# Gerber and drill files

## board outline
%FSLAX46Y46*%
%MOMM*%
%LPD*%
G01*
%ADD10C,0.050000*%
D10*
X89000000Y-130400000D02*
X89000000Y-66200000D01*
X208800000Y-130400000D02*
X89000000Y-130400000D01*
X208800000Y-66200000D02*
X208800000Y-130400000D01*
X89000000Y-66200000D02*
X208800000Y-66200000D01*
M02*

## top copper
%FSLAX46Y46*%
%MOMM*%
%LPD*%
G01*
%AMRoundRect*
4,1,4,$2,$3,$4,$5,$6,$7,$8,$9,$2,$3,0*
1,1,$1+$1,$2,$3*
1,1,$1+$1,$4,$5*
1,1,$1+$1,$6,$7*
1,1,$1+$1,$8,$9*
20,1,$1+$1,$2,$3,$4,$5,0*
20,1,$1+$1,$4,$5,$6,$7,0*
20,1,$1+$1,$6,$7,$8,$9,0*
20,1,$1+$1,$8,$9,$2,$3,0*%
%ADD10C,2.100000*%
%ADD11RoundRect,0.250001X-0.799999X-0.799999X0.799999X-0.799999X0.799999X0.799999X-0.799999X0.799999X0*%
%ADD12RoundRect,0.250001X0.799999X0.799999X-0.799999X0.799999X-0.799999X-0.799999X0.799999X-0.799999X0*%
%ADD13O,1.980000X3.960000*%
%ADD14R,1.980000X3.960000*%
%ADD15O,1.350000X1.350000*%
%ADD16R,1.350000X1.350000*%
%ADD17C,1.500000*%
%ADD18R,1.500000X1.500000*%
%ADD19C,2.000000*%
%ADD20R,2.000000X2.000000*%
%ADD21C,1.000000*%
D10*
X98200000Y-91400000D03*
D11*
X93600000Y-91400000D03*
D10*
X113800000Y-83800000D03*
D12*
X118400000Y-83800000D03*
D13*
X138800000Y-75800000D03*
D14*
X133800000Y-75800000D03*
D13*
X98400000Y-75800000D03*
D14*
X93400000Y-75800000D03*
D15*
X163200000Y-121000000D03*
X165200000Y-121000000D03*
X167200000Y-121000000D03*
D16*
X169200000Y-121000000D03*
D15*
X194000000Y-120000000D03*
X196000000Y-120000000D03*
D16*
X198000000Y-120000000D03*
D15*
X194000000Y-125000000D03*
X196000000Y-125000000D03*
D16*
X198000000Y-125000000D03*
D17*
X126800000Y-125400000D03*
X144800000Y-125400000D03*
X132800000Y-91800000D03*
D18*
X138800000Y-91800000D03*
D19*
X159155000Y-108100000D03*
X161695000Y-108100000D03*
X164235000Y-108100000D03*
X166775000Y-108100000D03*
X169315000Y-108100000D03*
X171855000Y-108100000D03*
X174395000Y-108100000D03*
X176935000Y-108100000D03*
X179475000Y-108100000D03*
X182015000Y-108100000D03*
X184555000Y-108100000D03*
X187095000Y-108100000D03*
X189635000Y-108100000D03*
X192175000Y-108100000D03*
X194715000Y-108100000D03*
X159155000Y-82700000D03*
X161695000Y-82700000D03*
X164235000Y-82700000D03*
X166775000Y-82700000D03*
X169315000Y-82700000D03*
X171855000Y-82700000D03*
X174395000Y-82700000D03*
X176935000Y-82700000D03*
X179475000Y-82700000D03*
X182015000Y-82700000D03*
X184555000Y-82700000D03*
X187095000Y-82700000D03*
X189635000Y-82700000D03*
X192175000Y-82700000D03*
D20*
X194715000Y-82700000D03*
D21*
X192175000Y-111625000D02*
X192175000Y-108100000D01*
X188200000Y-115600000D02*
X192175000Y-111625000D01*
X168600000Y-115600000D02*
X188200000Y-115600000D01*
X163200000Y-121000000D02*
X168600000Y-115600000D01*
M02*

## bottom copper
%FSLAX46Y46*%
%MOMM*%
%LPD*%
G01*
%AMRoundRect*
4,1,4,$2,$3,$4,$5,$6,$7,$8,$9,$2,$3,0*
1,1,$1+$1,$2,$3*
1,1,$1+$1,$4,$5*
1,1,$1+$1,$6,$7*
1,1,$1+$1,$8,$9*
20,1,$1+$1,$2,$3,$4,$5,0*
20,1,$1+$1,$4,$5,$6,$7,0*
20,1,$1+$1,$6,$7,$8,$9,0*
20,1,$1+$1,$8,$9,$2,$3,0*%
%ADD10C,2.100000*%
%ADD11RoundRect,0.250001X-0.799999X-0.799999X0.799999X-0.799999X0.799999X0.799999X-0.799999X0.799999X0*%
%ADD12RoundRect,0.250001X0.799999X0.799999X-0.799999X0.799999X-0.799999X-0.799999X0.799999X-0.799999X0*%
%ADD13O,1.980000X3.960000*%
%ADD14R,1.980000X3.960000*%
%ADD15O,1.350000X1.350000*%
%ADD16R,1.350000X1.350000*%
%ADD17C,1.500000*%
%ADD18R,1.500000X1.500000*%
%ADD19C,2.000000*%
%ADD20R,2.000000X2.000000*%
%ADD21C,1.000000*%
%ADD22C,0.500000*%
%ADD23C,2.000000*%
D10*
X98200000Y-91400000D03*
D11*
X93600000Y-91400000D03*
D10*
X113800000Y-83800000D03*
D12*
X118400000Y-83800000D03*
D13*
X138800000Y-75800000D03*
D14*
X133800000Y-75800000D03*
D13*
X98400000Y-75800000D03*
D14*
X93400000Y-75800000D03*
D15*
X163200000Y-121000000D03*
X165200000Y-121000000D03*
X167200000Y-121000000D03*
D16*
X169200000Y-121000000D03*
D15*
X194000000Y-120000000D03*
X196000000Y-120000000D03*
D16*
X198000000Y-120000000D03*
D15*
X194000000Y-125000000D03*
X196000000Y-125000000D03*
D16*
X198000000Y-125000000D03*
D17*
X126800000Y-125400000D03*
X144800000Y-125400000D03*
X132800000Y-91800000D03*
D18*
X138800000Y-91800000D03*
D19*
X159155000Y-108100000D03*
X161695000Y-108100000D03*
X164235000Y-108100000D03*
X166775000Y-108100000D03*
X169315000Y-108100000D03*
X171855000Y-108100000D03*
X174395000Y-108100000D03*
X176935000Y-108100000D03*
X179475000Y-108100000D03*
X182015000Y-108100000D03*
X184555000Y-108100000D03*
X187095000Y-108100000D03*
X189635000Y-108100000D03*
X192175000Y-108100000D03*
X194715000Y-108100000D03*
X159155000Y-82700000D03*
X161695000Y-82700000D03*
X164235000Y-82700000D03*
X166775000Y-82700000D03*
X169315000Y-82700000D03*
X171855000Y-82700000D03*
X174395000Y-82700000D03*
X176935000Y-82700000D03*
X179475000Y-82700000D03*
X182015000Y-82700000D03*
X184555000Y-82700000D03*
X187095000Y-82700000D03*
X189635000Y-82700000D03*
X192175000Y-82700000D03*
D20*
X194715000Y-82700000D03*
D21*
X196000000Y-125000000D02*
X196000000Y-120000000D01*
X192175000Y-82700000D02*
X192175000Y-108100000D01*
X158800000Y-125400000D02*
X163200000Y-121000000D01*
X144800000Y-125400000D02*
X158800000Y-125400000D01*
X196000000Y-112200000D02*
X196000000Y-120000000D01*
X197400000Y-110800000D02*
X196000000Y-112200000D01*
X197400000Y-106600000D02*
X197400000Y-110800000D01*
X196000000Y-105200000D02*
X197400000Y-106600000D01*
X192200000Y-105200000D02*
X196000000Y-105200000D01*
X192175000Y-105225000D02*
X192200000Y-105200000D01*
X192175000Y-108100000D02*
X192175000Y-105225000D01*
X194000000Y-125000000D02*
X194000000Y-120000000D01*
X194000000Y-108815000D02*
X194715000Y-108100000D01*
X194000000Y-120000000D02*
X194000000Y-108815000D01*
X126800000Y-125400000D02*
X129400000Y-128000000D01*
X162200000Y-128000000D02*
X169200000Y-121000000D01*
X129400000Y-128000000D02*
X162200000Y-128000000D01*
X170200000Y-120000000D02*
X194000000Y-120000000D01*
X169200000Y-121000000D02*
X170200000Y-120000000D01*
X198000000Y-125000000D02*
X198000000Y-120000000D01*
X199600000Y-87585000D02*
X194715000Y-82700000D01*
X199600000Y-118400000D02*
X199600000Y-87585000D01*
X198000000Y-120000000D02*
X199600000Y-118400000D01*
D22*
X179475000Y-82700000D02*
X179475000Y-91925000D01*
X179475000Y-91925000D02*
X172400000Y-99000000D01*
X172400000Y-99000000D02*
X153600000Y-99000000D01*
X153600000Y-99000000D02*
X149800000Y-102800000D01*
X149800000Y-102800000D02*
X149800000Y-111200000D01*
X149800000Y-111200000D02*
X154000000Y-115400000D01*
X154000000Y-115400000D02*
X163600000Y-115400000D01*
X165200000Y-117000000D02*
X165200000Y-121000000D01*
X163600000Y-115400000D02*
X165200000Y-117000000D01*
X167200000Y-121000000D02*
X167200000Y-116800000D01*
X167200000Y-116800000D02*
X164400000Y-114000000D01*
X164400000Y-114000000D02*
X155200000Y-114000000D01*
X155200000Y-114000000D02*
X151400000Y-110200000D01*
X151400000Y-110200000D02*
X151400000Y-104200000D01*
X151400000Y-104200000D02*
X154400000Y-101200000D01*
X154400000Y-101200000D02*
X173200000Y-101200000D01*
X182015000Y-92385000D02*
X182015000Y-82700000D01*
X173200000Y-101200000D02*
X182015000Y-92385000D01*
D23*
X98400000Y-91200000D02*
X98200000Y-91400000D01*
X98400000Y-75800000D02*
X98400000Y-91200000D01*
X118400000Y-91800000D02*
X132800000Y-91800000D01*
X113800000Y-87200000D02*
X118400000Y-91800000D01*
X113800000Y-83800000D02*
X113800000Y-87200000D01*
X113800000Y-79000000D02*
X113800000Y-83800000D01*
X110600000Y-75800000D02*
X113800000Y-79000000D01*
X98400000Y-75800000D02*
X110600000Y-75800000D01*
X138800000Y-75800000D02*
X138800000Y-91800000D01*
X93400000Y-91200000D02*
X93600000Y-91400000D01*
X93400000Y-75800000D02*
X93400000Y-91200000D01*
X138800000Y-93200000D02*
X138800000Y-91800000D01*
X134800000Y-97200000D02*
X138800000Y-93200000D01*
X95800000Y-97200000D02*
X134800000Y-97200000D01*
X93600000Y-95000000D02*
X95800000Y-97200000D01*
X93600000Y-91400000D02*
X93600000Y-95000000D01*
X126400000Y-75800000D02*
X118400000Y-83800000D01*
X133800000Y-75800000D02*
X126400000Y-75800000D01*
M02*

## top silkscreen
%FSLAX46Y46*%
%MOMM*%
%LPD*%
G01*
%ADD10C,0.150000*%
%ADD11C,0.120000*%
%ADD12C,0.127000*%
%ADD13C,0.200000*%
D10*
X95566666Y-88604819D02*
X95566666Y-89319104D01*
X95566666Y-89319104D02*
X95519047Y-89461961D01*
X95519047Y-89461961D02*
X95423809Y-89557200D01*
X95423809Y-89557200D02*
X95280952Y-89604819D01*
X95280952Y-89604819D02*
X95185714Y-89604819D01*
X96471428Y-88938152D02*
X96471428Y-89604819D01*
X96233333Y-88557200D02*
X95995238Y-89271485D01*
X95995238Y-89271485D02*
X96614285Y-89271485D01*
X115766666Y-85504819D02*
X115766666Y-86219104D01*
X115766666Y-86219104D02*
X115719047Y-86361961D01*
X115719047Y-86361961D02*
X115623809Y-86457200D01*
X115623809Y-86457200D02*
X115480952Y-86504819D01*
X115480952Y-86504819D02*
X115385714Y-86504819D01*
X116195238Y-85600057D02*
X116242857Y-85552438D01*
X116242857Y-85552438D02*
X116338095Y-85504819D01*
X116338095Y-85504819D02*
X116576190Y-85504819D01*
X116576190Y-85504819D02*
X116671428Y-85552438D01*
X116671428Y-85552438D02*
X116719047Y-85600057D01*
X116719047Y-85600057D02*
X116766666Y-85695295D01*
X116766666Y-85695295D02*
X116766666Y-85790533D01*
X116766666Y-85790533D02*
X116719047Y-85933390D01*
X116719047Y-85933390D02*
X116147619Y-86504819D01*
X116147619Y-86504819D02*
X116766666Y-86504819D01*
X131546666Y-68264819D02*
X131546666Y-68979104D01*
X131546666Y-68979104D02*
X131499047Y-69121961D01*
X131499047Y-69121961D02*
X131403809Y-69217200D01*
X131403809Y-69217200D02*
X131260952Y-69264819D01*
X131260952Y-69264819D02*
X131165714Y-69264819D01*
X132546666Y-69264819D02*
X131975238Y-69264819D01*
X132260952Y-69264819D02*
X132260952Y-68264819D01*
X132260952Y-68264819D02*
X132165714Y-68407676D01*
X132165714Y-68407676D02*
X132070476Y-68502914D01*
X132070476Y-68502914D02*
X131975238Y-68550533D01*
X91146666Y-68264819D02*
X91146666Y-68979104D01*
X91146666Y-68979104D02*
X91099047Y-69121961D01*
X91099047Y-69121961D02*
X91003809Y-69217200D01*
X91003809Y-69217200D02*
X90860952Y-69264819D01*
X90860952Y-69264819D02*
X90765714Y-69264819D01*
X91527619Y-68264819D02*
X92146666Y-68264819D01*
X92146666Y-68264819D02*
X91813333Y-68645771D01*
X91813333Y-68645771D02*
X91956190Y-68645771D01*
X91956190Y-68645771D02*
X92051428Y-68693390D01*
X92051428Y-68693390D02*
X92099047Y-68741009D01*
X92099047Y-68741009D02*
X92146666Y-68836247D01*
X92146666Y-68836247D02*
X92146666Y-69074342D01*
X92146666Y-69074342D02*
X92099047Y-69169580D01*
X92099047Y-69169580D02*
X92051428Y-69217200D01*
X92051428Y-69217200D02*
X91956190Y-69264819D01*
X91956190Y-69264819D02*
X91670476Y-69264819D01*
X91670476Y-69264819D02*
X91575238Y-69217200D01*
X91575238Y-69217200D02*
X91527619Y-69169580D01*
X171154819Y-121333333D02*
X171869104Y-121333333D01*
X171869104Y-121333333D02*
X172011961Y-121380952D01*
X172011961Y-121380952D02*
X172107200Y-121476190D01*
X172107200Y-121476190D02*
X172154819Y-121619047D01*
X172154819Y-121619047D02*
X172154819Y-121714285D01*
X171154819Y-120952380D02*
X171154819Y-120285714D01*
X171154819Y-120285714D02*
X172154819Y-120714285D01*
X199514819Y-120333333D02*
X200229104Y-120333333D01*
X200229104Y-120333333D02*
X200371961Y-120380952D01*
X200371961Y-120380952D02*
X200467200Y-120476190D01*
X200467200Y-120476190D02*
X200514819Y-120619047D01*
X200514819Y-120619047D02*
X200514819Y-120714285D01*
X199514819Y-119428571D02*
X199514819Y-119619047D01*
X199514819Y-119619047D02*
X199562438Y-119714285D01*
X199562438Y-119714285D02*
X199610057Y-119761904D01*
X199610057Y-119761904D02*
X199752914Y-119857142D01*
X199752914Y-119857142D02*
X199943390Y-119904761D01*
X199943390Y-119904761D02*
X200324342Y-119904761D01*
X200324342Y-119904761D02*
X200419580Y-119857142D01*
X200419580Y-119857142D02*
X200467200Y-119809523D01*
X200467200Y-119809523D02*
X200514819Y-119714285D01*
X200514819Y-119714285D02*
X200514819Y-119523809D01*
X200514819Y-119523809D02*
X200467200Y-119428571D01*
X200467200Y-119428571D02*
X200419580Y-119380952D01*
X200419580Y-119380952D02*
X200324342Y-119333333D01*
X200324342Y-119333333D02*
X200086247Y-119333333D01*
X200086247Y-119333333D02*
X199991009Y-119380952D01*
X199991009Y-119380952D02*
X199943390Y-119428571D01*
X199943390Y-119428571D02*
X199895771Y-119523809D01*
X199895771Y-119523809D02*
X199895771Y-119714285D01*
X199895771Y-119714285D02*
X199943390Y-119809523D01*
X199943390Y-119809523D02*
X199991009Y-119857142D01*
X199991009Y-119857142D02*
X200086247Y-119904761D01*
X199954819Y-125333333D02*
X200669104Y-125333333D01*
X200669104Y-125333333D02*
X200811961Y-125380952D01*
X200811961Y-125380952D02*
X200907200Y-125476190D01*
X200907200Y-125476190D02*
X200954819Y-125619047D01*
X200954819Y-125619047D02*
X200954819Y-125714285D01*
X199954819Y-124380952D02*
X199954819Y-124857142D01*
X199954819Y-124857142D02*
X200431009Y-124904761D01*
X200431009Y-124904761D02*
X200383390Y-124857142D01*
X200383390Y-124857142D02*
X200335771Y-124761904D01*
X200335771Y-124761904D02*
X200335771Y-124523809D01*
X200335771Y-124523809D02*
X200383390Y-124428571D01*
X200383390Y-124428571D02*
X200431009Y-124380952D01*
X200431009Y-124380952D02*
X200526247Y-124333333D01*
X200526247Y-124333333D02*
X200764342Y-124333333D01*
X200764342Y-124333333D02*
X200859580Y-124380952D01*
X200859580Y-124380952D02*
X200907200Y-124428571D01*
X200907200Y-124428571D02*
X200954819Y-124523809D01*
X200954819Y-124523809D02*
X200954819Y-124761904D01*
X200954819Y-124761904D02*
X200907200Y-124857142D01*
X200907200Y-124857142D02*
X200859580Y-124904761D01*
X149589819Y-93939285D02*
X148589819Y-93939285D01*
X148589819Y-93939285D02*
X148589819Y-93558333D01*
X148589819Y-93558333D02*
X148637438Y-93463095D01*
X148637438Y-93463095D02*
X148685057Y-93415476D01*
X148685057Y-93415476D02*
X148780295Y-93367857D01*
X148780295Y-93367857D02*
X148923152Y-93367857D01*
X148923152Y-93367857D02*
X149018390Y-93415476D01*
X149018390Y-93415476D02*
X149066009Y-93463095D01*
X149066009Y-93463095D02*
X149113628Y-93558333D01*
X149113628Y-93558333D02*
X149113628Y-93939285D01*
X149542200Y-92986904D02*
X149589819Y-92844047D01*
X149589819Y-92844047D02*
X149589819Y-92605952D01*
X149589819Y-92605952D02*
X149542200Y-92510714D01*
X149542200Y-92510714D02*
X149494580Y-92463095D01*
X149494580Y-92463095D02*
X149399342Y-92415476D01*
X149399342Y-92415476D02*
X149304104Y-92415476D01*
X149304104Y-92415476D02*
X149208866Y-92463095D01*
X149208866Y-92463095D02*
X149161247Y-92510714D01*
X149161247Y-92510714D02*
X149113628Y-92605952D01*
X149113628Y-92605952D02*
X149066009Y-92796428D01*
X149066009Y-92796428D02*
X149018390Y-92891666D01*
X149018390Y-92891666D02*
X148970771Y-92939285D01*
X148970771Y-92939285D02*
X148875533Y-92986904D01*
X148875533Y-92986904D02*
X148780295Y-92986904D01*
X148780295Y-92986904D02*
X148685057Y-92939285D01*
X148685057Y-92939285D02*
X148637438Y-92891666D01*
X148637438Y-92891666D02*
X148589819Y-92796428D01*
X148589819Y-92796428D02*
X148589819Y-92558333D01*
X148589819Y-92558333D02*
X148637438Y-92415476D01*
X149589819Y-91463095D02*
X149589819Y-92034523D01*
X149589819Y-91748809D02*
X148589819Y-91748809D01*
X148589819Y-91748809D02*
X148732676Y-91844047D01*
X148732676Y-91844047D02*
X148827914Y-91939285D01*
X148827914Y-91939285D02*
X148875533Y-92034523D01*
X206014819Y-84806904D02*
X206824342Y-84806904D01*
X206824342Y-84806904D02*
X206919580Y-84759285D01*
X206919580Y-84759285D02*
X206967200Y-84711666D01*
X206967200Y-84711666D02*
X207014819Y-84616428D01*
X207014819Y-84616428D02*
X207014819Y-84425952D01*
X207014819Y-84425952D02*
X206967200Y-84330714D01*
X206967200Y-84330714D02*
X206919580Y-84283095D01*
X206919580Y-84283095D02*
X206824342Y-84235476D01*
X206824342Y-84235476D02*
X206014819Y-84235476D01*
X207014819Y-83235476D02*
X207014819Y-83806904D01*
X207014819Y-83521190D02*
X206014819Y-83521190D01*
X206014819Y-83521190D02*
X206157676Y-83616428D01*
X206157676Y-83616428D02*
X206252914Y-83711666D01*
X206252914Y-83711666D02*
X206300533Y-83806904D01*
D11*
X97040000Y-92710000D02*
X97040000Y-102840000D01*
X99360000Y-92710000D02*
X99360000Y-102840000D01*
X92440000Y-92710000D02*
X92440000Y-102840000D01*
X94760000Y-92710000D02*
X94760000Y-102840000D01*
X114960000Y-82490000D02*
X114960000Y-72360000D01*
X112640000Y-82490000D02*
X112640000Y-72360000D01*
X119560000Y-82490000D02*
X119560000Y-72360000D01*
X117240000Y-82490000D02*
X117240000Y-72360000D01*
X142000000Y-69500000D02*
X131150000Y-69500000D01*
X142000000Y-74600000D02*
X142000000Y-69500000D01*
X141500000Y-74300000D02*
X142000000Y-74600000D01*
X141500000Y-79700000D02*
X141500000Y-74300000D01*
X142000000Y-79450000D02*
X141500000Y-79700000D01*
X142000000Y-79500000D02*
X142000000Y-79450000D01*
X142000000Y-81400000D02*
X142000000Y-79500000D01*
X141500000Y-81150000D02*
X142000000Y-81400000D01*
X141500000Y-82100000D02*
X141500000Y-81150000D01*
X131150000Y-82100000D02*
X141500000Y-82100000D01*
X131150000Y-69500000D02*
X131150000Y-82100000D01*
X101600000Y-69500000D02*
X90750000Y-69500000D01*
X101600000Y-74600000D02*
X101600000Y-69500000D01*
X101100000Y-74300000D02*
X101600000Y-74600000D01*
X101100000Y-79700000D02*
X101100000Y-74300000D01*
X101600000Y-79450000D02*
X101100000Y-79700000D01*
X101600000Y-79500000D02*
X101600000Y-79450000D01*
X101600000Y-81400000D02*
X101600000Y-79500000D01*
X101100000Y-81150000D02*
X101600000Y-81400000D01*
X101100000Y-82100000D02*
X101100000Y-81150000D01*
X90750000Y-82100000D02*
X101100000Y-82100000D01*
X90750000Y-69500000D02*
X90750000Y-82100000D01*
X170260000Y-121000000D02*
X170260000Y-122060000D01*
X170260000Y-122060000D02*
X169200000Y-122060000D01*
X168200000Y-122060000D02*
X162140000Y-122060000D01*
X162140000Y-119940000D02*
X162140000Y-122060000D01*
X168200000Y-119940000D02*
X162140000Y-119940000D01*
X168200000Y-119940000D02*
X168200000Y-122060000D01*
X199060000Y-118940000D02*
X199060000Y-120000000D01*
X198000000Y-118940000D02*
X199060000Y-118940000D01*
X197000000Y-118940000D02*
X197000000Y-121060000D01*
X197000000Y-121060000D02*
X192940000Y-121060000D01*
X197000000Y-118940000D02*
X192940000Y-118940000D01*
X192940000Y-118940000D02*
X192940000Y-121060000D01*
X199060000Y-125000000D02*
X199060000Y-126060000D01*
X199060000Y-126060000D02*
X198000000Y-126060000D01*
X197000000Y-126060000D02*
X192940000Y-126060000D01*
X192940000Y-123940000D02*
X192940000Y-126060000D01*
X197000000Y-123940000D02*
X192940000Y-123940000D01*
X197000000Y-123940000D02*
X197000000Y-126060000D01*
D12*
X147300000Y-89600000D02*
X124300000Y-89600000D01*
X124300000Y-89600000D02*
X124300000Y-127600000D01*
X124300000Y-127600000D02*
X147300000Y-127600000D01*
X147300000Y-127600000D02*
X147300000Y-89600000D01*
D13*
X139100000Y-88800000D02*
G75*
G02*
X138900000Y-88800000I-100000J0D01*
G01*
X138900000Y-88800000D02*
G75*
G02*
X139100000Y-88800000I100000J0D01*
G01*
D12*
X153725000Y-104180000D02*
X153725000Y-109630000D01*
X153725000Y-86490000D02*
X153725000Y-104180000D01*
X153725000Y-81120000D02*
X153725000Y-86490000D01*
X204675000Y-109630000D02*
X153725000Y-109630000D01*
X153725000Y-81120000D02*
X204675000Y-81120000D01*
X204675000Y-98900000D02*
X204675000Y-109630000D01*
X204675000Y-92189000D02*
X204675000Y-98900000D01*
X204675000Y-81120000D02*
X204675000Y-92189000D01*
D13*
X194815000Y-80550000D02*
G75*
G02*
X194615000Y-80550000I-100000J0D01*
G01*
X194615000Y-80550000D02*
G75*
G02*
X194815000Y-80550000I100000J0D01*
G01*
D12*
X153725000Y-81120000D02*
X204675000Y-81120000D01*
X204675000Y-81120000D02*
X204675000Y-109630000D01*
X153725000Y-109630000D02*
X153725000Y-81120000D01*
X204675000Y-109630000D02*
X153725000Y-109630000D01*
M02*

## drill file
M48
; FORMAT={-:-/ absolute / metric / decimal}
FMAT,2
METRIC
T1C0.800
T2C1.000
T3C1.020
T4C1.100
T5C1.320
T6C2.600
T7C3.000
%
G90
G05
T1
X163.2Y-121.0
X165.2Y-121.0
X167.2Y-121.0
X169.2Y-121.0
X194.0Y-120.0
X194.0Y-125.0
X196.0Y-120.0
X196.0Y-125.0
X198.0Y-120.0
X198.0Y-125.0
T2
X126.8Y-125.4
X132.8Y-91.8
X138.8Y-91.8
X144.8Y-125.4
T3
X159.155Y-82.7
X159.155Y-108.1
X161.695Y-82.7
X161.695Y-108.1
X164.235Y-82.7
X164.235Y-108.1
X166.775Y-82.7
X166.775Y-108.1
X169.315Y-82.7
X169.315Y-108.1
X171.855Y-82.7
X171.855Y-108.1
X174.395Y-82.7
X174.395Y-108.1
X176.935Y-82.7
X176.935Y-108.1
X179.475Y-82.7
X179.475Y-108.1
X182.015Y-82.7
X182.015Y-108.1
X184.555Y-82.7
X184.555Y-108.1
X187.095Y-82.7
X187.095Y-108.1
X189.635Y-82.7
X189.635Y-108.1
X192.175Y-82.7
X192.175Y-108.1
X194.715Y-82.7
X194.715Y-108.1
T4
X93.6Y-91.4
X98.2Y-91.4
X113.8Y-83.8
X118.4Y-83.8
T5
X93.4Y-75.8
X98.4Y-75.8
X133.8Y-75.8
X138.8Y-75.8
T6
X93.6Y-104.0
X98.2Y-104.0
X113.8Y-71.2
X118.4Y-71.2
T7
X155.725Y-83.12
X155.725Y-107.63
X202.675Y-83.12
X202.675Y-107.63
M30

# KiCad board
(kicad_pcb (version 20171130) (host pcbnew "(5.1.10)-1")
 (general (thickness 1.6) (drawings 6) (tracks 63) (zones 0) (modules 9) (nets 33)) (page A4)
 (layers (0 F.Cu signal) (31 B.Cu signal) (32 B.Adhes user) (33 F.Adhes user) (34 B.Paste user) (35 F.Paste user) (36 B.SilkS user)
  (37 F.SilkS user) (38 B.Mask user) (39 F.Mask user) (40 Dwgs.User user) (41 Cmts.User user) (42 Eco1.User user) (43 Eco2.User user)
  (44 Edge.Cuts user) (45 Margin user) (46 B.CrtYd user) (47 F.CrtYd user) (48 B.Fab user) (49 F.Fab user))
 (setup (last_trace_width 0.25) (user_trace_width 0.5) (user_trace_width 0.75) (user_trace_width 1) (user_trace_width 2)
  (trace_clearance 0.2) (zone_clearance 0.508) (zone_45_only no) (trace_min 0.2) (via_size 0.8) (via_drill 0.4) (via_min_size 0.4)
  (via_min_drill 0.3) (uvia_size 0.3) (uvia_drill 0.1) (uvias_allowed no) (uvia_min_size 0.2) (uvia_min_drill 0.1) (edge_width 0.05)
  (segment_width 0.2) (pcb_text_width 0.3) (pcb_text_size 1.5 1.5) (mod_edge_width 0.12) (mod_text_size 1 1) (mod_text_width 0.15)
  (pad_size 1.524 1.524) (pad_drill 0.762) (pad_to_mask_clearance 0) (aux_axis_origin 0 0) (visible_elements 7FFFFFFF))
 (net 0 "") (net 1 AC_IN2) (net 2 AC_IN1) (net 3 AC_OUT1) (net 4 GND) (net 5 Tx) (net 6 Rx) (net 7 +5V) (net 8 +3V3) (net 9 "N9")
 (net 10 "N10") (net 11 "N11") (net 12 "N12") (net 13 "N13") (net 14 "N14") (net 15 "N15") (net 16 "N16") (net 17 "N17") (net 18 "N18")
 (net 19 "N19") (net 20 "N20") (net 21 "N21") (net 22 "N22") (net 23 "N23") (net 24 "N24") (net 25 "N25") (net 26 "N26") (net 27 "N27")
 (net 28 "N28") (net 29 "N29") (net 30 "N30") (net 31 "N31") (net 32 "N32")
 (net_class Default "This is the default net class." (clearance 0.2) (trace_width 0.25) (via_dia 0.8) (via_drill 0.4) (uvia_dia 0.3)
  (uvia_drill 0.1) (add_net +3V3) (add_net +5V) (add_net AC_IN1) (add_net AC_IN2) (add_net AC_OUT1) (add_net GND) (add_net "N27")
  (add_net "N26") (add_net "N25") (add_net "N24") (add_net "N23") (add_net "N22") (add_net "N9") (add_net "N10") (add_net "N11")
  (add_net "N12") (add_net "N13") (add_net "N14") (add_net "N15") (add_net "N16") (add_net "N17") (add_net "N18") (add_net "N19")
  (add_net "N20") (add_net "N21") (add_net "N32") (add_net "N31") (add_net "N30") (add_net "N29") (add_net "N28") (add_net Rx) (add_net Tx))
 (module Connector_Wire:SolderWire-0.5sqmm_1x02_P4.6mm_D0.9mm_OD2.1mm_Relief (layer F.Cu) (at 93.6 91.4)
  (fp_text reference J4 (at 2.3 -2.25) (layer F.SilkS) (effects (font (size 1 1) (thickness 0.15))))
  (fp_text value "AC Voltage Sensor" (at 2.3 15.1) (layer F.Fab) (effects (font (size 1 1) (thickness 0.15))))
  (fp_line (start 3.44 1.31) (end 3.44 11.44) (layer F.SilkS) (width 0.12))
  (fp_line (start 5.76 1.31) (end 5.76 11.44) (layer F.SilkS) (width 0.12))
  (fp_line (start -1.16 1.31) (end -1.16 11.44) (layer F.SilkS) (width 0.12))
  (fp_line (start 1.16 1.31) (end 1.16 11.44) (layer F.SilkS) (width 0.12))
  (pad "" np_thru_hole circle (at 4.6 12.6) (size 2.6 2.6) (drill 2.6) (layers *.Cu *.Mask))
  (pad "" np_thru_hole circle (at 0 12.6) (size 2.6 2.6) (drill 2.6) (layers *.Cu *.Mask))
  (pad 2 thru_hole circle (at 4.6 0) (size 2.1 2.1) (drill 1.1) (layers *.Cu *.Mask) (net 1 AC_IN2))
  (pad 1 thru_hole roundrect (at 0 0) (size 2.1 2.1) (drill 1.1) (layers *.Cu *.Mask) (roundrect_rratio 0.119048) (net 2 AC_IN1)))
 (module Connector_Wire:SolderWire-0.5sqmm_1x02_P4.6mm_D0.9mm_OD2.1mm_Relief (layer F.Cu) (at 118.4 83.8 180)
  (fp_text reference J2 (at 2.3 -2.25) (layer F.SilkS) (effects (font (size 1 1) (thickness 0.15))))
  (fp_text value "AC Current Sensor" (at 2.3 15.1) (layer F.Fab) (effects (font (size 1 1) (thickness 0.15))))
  (fp_line (start 3.44 1.31) (end 3.44 11.44) (layer F.SilkS) (width 0.12))
  (fp_line (start 5.76 1.31) (end 5.76 11.44) (layer F.SilkS) (width 0.12))
  (fp_line (start -1.16 1.31) (end -1.16 11.44) (layer F.SilkS) (width 0.12))
  (fp_line (start 1.16 1.31) (end 1.16 11.44) (layer F.SilkS) (width 0.12))
  (pad "" np_thru_hole circle (at 4.6 12.6 180) (size 2.6 2.6) (drill 2.6) (layers *.Cu *.Mask))
  (pad "" np_thru_hole circle (at 0 12.6 180) (size 2.6 2.6) (drill 2.6) (layers *.Cu *.Mask))
  (pad 2 thru_hole circle (at 4.6 0 180) (size 2.1 2.1) (drill 1.1) (layers *.Cu *.Mask) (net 1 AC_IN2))
  (pad 1 thru_hole roundrect (at 0 0 180) (size 2.1 2.1) (drill 1.1) (layers *.Cu *.Mask) (roundrect_rratio 0.119048) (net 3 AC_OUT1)))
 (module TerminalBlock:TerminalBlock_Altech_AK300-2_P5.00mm (layer F.Cu) (at 133.8 75.8)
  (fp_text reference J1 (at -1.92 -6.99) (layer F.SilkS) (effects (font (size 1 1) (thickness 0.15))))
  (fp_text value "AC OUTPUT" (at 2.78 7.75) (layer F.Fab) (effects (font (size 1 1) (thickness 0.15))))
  (fp_line (start 8.2 -6.3) (end -2.65 -6.3) (layer F.SilkS) (width 0.12))
  (fp_line (start 8.2 -1.2) (end 8.2 -6.3) (layer F.SilkS) (width 0.12))
  (fp_line (start 7.7 -1.5) (end 8.2 -1.2) (layer F.SilkS) (width 0.12))
  (fp_line (start 7.7 3.9) (end 7.7 -1.5) (layer F.SilkS) (width 0.12))
  (fp_line (start 8.2 3.65) (end 7.7 3.9) (layer F.SilkS) (width 0.12))
  (fp_line (start 8.2 3.7) (end 8.2 3.65) (layer F.SilkS) (width 0.12))
  (fp_line (start 8.2 5.6) (end 8.2 3.7) (layer F.SilkS) (width 0.12))
  (fp_line (start 7.7 5.35) (end 8.2 5.6) (layer F.SilkS) (width 0.12))
  (fp_line (start 7.7 6.3) (end 7.7 5.35) (layer F.SilkS) (width 0.12))
  (fp_line (start -2.65 6.3) (end 7.7 6.3) (layer F.SilkS) (width 0.12))
  (fp_line (start -2.65 -6.3) (end -2.65 6.3) (layer F.SilkS) (width 0.12))
  (pad 2 thru_hole oval (at 5 0) (size 1.98 3.96) (drill 1.32) (layers *.Cu *.Mask) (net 2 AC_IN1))
  (pad 1 thru_hole rect (at 0 0) (size 1.98 3.96) (drill 1.32) (layers *.Cu *.Mask) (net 3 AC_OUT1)))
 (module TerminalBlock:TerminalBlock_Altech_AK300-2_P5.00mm (layer F.Cu) (at 93.4 75.8)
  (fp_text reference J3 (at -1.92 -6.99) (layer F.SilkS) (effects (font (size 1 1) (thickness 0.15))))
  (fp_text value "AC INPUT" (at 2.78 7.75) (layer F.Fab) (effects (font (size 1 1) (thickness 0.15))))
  (fp_line (start 8.2 -6.3) (end -2.65 -6.3) (layer F.SilkS) (width 0.12))
  (fp_line (start 8.2 -1.2) (end 8.2 -6.3) (layer F.SilkS) (width 0.12))
  (fp_line (start 7.7 -1.5) (end 8.2 -1.2) (layer F.SilkS) (width 0.12))
  (fp_line (start 7.7 3.9) (end 7.7 -1.5) (layer F.SilkS) (width 0.12))
  (fp_line (start 8.2 3.65) (end 7.7 3.9) (layer F.SilkS) (width 0.12))
  (fp_line (start 8.2 3.7) (end 8.2 3.65) (layer F.SilkS) (width 0.12))
  (fp_line (start 8.2 5.6) (end 8.2 3.7) (layer F.SilkS) (width 0.12))
  (fp_line (start 7.7 5.35) (end 8.2 5.6) (layer F.SilkS) (width 0.12))
  (fp_line (start 7.7 6.3) (end 7.7 5.35) (layer F.SilkS) (width 0.12))
  (fp_line (start -2.65 6.3) (end 7.7 6.3) (layer F.SilkS) (width 0.12))
  (fp_line (start -2.65 -6.3) (end -2.65 6.3) (layer F.SilkS) (width 0.12))
  (pad 2 thru_hole oval (at 5 0) (size 1.98 3.96) (drill 1.32) (layers *.Cu *.Mask) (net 1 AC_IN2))
  (pad 1 thru_hole rect (at 0 0) (size 1.98 3.96) (drill 1.32) (layers *.Cu *.Mask) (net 2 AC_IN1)))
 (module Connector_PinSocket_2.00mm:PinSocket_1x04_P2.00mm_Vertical (layer F.Cu) (at 169.2 121 270)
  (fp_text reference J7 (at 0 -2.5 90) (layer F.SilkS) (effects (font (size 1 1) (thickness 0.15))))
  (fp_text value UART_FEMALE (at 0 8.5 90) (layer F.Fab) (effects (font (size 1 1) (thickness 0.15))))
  (fp_line (start 0 -1.06) (end 1.06 -1.06) (layer F.SilkS) (width 0.12))
  (fp_line (start 1.06 -1.06) (end 1.06 0) (layer F.SilkS) (width 0.12))
  (fp_line (start 1.06 1) (end 1.06 7.06) (layer F.SilkS) (width 0.12))
  (fp_line (start -1.06 7.06) (end 1.06 7.06) (layer F.SilkS) (width 0.12))
  (fp_line (start -1.06 1) (end -1.06 7.06) (layer F.SilkS) (width 0.12))
  (fp_line (start -1.06 1) (end 1.06 1) (layer F.SilkS) (width 0.12))
  (pad 4 thru_hole oval (at 0 6 270) (size 1.35 1.35) (drill 0.8) (layers *.Cu *.Mask) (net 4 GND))
  (pad 3 thru_hole oval (at 0 4 270) (size 1.35 1.35) (drill 0.8) (layers *.Cu *.Mask) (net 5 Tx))
  (pad 2 thru_hole oval (at 0 2 270) (size 1.35 1.35) (drill 0.8) (layers *.Cu *.Mask) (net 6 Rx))
  (pad 1 thru_hole rect (at 0 0 270) (size 1.35 1.35) (drill 0.8) (layers *.Cu *.Mask) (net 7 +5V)))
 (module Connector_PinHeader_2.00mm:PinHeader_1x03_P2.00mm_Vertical (layer F.Cu) (at 198 120 270)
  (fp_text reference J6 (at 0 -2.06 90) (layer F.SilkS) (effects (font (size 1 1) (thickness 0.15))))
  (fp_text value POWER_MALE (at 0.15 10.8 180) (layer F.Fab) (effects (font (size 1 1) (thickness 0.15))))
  (fp_line (start -1.06 -1.06) (end 0 -1.06) (layer F.SilkS) (width 0.12))
  (fp_line (start -1.06 0) (end -1.06 -1.06) (layer F.SilkS) (width 0.12))
  (fp_line (start -1.06 1) (end 1.06 1) (layer F.SilkS) (width 0.12))
  (fp_line (start 1.06 1) (end 1.06 5.06) (layer F.SilkS) (width 0.12))
  (fp_line (start -1.06 1) (end -1.06 5.06) (layer F.SilkS) (width 0.12))
  (fp_line (start -1.06 5.06) (end 1.06 5.06) (layer F.SilkS) (width 0.12))
  (pad 3 thru_hole oval (at 0 4 270) (size 1.35 1.35) (drill 0.8) (layers *.Cu *.Mask) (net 7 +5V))
  (pad 2 thru_hole oval (at 0 2 270) (size 1.35 1.35) (drill 0.8) (layers *.Cu *.Mask) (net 4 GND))
  (pad 1 thru_hole rect (at 0 0 270) (size 1.35 1.35) (drill 0.8) (layers *.Cu *.Mask) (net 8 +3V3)))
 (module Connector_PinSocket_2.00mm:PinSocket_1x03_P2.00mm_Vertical (layer F.Cu) (at 198 125 270)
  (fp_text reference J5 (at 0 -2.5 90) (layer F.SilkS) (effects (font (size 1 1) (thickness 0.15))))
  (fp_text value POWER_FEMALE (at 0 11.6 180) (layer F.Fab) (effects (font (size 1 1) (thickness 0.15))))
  (fp_line (start 0 -1.06) (end 1.06 -1.06) (layer F.SilkS) (width 0.12))
  (fp_line (start 1.06 -1.06) (end 1.06 0) (layer F.SilkS) (width 0.12))
  (fp_line (start 1.06 1) (end 1.06 5.06) (layer F.SilkS) (width 0.12))
  (fp_line (start -1.06 5.06) (end 1.06 5.06) (layer F.SilkS) (width 0.12))
  (fp_line (start -1.06 1) (end -1.06 5.06) (layer F.SilkS) (width 0.12))
  (fp_line (start -1.06 1) (end 1.06 1) (layer F.SilkS) (width 0.12))
  (pad 3 thru_hole oval (at 0 4 270) (size 1.35 1.35) (drill 0.8) (layers *.Cu *.Mask) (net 7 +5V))
  (pad 2 thru_hole oval (at 0 2 270) (size 1.35 1.35) (drill 0.8) (layers *.Cu *.Mask) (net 4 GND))
  (pad 1 thru_hole rect (at 0 0 270) (size 1.35 1.35) (drill 0.8) (layers *.Cu *.Mask) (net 8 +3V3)))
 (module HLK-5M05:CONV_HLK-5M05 (layer F.Cu) (at 135.8 108.6 270)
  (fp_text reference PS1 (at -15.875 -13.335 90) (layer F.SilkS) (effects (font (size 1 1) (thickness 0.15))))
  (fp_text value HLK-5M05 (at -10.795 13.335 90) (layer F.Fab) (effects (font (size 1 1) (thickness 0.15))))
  (fp_line (start -19 -11.5) (end -19 11.5) (layer F.SilkS) (width 0.127))
  (fp_line (start -19 11.5) (end 19 11.5) (layer F.SilkS) (width 0.127))
  (fp_line (start 19 11.5) (end 19 -11.5) (layer F.SilkS) (width 0.127))
  (fp_line (start 19 -11.5) (end -19 -11.5) (layer F.SilkS) (width 0.127))
  (fp_circle (center -19.8 -3.2) (end -19.7 -3.2) (layer F.SilkS) (width 0.2))
  (pad 4 thru_hole circle (at 16.8 9 270) (size 1.5 1.5) (drill 1) (layers *.Cu *.Mask) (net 7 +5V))
  (pad 3 thru_hole circle (at 16.8 -9 270) (size 1.5 1.5) (drill 1) (layers *.Cu *.Mask) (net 4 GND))
  (pad 2 thru_hole circle (at -16.8 3 270) (size 1.5 1.5) (drill 1) (layers *.Cu *.Mask) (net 1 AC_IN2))
  (pad 1 thru_hole rect (at -16.8 -3 270) (size 1.5 1.5) (drill 1) (layers *.Cu *.Mask) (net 2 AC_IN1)))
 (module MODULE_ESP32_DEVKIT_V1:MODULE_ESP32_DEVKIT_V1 (layer F.Cu) (at 179.2 95.4 270)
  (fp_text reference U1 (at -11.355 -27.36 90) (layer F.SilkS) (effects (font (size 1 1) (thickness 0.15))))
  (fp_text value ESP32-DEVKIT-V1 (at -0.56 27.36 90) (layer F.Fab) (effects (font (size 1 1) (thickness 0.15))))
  (fp_line (start 8.78 25.475) (end 14.23 25.475) (layer F.SilkS) (width 0.127))
  (fp_line (start -8.91 25.475) (end 8.78 25.475) (layer F.SilkS) (width 0.127))
  (fp_line (start -14.28 25.475) (end -8.91 25.475) (layer F.SilkS) (width 0.127))
  (fp_line (start 14.23 -25.475) (end 14.23 25.475) (layer F.SilkS) (width 0.127))
  (fp_line (start -14.28 25.475) (end -14.28 -25.475) (layer F.SilkS) (width 0.127))
  (fp_line (start 3.5 -25.475) (end 14.23 -25.475) (layer F.SilkS) (width 0.127))
  (fp_line (start -3.211 -25.475) (end 3.5 -25.475) (layer F.SilkS) (width 0.127))
  (fp_line (start -14.28 -25.475) (end -3.211 -25.475) (layer F.SilkS) (width 0.127))
  (fp_circle (center -14.85 -15.515) (end -14.75 -15.515) (layer F.SilkS) (width 0.2))
  (fp_line (start -14.28 25.475) (end -14.28 -25.475) (layer F.SilkS) (width 0.127))
  (fp_line (start -14.28 -25.475) (end 14.23 -25.475) (layer F.SilkS) (width 0.127))
  (fp_line (start 14.23 25.475) (end -14.28 25.475) (layer F.SilkS) (width 0.127))
  (fp_line (start 14.23 -25.475) (end 14.23 25.475) (layer F.SilkS) (width 0.127))
  (pad None np_thru_hole circle (at -12.28 -23.475 270) (size 3 3) (drill 3) (layers *.Cu *.Mask))
  (pad None np_thru_hole circle (at 12.23 -23.475 270) (size 3 3) (drill 3) (layers *.Cu *.Mask))
  (pad None np_thru_hole circle (at 12.23 23.475 270) (size 3 3) (drill 3) (layers *.Cu *.Mask))
  (pad None np_thru_hole circle (at -12.28 23.475 270) (size 3 3) (drill 3) (layers *.Cu *.Mask))
  (pad 16 thru_hole circle (at 12.7 20.045 270) (size 2 2) (drill 1.02) (layers *.Cu *.Mask) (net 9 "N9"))
  (pad 17 thru_hole circle (at 12.7 17.505 270) (size 2 2) (drill 1.02) (layers *.Cu *.Mask) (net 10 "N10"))
  (pad 18 thru_hole circle (at 12.7 14.965 270) (size 2 2) (drill 1.02) (layers *.Cu *.Mask) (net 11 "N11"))
  (pad 19 thru_hole circle (at 12.7 12.425 270) (size 2 2) (drill 1.02) (layers *.Cu *.Mask) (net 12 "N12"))
  (pad 20 thru_hole circle (at 12.7 9.885 270) (size 2 2) (drill 1.02) (layers *.Cu *.Mask) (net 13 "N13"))
  (pad 21 thru_hole circle (at 12.7 7.345 270) (size 2 2) (drill 1.02) (layers *.Cu *.Mask) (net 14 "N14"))
  (pad 22 thru_hole circle (at 12.7 4.805 270) (size 2 2) (drill 1.02) (layers *.Cu *.Mask) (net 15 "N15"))
  (pad 23 thru_hole circle (at 12.7 2.265 270) (size 2 2) (drill 1.02) (layers *.Cu *.Mask) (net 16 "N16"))
  (pad 24 thru_hole circle (at 12.7 -0.275 270) (size 2 2) (drill 1.02) (layers *.Cu *.Mask) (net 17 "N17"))
  (pad 25 thru_hole circle (at 12.7 -2.815 270) (size 2 2) (drill 1.02) (layers *.Cu *.Mask) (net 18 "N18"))
  (pad 26 thru_hole circle (at 12.7 -5.355 270) (size 2 2) (drill 1.02) (layers *.Cu *.Mask) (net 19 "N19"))
  (pad 27 thru_hole circle (at 12.7 -7.895 270) (size 2 2) (drill 1.02) (layers *.Cu *.Mask) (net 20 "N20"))
  (pad 28 thru_hole circle (at 12.7 -10.435 270) (size 2 2) (drill 1.02) (layers *.Cu *.Mask) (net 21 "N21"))
  (pad 29 thru_hole circle (at 12.7 -12.975 270) (size 2 2) (drill 1.02) (layers *.Cu *.Mask) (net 4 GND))
  (pad 30 thru_hole circle (at 12.7 -15.515 270) (size 2 2) (drill 1.02) (layers *.Cu *.Mask) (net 7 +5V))
  (pad 15 thru_hole circle (at -12.7 20.045 270) (size 2 2) (drill 1.02) (layers *.Cu *.Mask) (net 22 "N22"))
  (pad 14 thru_hole circle (at -12.7 17.505 270) (size 2 2) (drill 1.02) (layers *.Cu *.Mask) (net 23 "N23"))
  (pad 13 thru_hole circle (at -12.7 14.965 270) (size 2 2) (drill 1.02) (layers *.Cu *.Mask) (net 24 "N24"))
  (pad 12 thru_hole circle (at -12.7 12.425 270) (size 2 2) (drill 1.02) (layers *.Cu *.Mask) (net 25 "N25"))
  (pad 11 thru_hole circle (at -12.7 9.885 270) (size 2 2) (drill 1.02) (layers *.Cu *.Mask) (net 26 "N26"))
  (pad 10 thru_hole circle (at -12.7 7.345 270) (size 2 2) (drill 1.02) (layers *.Cu *.Mask) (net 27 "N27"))
  (pad 9 thru_hole circle (at -12.7 4.805 270) (size 2 2) (drill 1.02) (layers *.Cu *.Mask) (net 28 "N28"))
  (pad 8 thru_hole circle (at -12.7 2.265 270) (size 2 2) (drill 1.02) (layers *.Cu *.Mask) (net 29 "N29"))
  (pad 7 thru_hole circle (at -12.7 -0.275 270) (size 2 2) (drill 1.02) (layers *.Cu *.Mask) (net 5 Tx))
  (pad 6 thru_hole circle (at -12.7 -2.815 270) (size 2 2) (drill 1.02) (layers *.Cu *.Mask) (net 6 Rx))
  (pad 5 thru_hole circle (at -12.7 -5.355 270) (size 2 2) (drill 1.02) (layers *.Cu *.Mask) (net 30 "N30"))
  (pad 4 thru_hole circle (at -12.7 -7.895 270) (size 2 2) (drill 1.02) (layers *.Cu *.Mask) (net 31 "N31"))
  (pad 3 thru_hole circle (at -12.7 -10.435 270) (size 2 2) (drill 1.02) (layers *.Cu *.Mask) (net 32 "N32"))
  (pad 2 thru_hole circle (at -12.7 -12.975 270) (size 2 2) (drill 1.02) (layers *.Cu *.Mask) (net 4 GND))
  (pad 1 thru_hole rect (at -12.7 -15.515 270) (size 2 2) (drill 1.02) (layers *.Cu *.Mask) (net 8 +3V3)))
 (gr_line (start 89 130.4) (end 89 66.2) (layer Edge.Cuts) (width 0.05))
 (gr_line (start 208.8 130.4) (end 89 130.4) (layer Edge.Cuts) (width 0.05))
 (gr_line (start 208.8 66.2) (end 208.8 130.4) (layer Edge.Cuts) (width 0.05))
 (gr_line (start 89 66.2) (end 208.8 66.2) (layer Edge.Cuts) (width 0.05))
 (segment (start 196 125) (end 196 120) (width 1) (layer B.Cu) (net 4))
 (segment (start 192.175 82.7) (end 192.175 108.1) (width 1) (layer B.Cu) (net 4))
 (segment (start 158.8 125.4) (end 163.2 121) (width 1) (layer B.Cu) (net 4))
 (segment (start 144.8 125.4) (end 158.8 125.4) (width 1) (layer B.Cu) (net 4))
 (segment (start 192.175 111.625) (end 192.175 108.1) (width 1) (layer F.Cu) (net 4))
 (segment (start 188.2 115.6) (end 192.175 111.625) (width 1) (layer F.Cu) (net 4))
 (segment (start 168.6 115.6) (end 188.2 115.6) (width 1) (layer F.Cu) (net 4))
 (segment (start 163.2 121) (end 168.6 115.6) (width 1) (layer F.Cu) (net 4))
 (segment (start 196 112.2) (end 196 120) (width 1) (layer B.Cu) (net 4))
 (segment (start 197.4 110.8) (end 196 112.2) (width 1) (layer B.Cu) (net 4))
 (segment (start 197.4 106.6) (end 197.4 110.8) (width 1) (layer B.Cu) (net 4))
 (segment (start 196 105.2) (end 197.4 106.6) (width 1) (layer B.Cu) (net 4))
 (segment (start 192.2 105.2) (end 196 105.2) (width 1) (layer B.Cu) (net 4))
 (segment (start 192.175 105.225) (end 192.2 105.2) (width 1) (layer B.Cu) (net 4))
 (segment (start 192.175 108.1) (end 192.175 105.225) (width 1) (layer B.Cu) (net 4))
 (segment (start 194 125) (end 194 120) (width 1) (layer B.Cu) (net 7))
 (segment (start 194 108.815) (end 194.715 108.1) (width 1) (layer B.Cu) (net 7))
 (segment (start 194 120) (end 194 108.815) (width 1) (layer B.Cu) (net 7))
 (segment (start 126.8 125.4) (end 129.4 128) (width 1) (layer B.Cu) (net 7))
 (segment (start 162.2 128) (end 169.2 121) (width 1) (layer B.Cu) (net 7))
 (segment (start 129.4 128) (end 162.2 128) (width 1) (layer B.Cu) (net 7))
 (segment (start 170.2 120) (end 194 120) (width 1) (layer B.Cu) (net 7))
 (segment (start 169.2 121) (end 170.2 120) (width 1) (layer B.Cu) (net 7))
 (segment (start 198 125) (end 198 120) (width 1) (layer B.Cu) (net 8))
 (segment (start 199.6 87.585) (end 194.715 82.7) (width 1) (layer B.Cu) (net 8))
 (segment (start 199.6 118.4) (end 199.6 87.585) (width 1) (layer B.Cu) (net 8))
 (segment (start 198 120) (end 199.6 118.4) (width 1) (layer B.Cu) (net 8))
 (segment (start 179.475 82.7) (end 179.475 91.925) (width 0.5) (layer B.Cu) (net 5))
 (segment (start 179.475 91.925) (end 172.4 99) (width 0.5) (layer B.Cu) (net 5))
 (segment (start 172.4 99) (end 153.6 99) (width 0.5) (layer B.Cu) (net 5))
 (segment (start 153.6 99) (end 149.8 102.8) (width 0.5) (layer B.Cu) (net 5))
 (segment (start 149.8 102.8) (end 149.8 111.2) (width 0.5) (layer B.Cu) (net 5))
 (segment (start 149.8 111.2) (end 154 115.4) (width 0.5) (layer B.Cu) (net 5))
 (segment (start 154 115.4) (end 163.6 115.4) (width 0.5) (layer B.Cu) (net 5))
 (segment (start 165.2 117) (end 165.2 121) (width 0.5) (layer B.Cu) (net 5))
 (segment (start 163.6 115.4) (end 165.2 117) (width 0.5) (layer B.Cu) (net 5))
 (segment (start 167.2 121) (end 167.2 116.8) (width 0.5) (layer B.Cu) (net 6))
 (segment (start 167.2 116.8) (end 164.4 114) (width 0.5) (layer B.Cu) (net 6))
 (segment (start 164.4 114) (end 155.2 114) (width 0.5) (layer B.Cu) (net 6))
 (segment (start 155.2 114) (end 151.4 110.2) (width 0.5) (layer B.Cu) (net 6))
 (segment (start 151.4 110.2) (end 151.4 104.2) (width 0.5) (layer B.Cu) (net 6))
 (segment (start 151.4 104.2) (end 154.4 101.2) (width 0.5) (layer B.Cu) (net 6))
 (segment (start 154.4 101.2) (end 173.2 101.2) (width 0.5) (layer B.Cu) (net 6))
 (segment (start 182.015 92.385) (end 182.015 82.7) (width 0.5) (layer B.Cu) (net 6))
 (segment (start 173.2 101.2) (end 182.015 92.385) (width 0.5) (layer B.Cu) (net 6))
 (segment (start 98.4 91.2) (end 98.2 91.4) (width 2) (layer B.Cu) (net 1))
 (segment (start 98.4 75.8) (end 98.4 91.2) (width 2) (layer B.Cu) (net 1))
 (segment (start 118.4 91.8) (end 132.8 91.8) (width 2) (layer B.Cu) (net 1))
 (segment (start 113.8 87.2) (end 118.4 91.8) (width 2) (layer B.Cu) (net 1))
 (segment (start 113.8 83.8) (end 113.8 87.2) (width 2) (layer B.Cu) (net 1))
 (segment (start 113.8 79) (end 113.8 83.8) (width 2) (layer B.Cu) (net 1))
 (segment (start 110.6 75.8) (end 113.8 79) (width 2) (layer B.Cu) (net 1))
 (segment (start 98.4 75.8) (end 110.6 75.8) (width 2) (layer B.Cu) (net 1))
 (segment (start 138.8 75.8) (end 138.8 91.8) (width 2) (layer B.Cu) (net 2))
 (segment (start 93.4 91.2) (end 93.6 91.4) (width 2) (layer B.Cu) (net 2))
 (segment (start 93.4 75.8) (end 93.4 91.2) (width 2) (layer B.Cu) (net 2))
 (segment (start 138.8 93.2) (end 138.8 91.8) (width 2) (layer B.Cu) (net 2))
 (segment (start 134.8 97.2) (end 138.8 93.2) (width 2) (layer B.Cu) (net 2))
 (segment (start 95.8 97.2) (end 134.8 97.2) (width 2) (layer B.Cu) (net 2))
 (segment (start 93.6 95) (end 95.8 97.2) (width 2) (layer B.Cu) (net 2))
 (segment (start 93.6 91.4) (end 93.6 95) (width 2) (layer B.Cu) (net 2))
 (segment (start 126.4 75.8) (end 118.4 83.8) (width 2) (layer B.Cu) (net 3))
 (segment (start 133.8 75.8) (end 126.4 75.8) (width 2) (layer B.Cu) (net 3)))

